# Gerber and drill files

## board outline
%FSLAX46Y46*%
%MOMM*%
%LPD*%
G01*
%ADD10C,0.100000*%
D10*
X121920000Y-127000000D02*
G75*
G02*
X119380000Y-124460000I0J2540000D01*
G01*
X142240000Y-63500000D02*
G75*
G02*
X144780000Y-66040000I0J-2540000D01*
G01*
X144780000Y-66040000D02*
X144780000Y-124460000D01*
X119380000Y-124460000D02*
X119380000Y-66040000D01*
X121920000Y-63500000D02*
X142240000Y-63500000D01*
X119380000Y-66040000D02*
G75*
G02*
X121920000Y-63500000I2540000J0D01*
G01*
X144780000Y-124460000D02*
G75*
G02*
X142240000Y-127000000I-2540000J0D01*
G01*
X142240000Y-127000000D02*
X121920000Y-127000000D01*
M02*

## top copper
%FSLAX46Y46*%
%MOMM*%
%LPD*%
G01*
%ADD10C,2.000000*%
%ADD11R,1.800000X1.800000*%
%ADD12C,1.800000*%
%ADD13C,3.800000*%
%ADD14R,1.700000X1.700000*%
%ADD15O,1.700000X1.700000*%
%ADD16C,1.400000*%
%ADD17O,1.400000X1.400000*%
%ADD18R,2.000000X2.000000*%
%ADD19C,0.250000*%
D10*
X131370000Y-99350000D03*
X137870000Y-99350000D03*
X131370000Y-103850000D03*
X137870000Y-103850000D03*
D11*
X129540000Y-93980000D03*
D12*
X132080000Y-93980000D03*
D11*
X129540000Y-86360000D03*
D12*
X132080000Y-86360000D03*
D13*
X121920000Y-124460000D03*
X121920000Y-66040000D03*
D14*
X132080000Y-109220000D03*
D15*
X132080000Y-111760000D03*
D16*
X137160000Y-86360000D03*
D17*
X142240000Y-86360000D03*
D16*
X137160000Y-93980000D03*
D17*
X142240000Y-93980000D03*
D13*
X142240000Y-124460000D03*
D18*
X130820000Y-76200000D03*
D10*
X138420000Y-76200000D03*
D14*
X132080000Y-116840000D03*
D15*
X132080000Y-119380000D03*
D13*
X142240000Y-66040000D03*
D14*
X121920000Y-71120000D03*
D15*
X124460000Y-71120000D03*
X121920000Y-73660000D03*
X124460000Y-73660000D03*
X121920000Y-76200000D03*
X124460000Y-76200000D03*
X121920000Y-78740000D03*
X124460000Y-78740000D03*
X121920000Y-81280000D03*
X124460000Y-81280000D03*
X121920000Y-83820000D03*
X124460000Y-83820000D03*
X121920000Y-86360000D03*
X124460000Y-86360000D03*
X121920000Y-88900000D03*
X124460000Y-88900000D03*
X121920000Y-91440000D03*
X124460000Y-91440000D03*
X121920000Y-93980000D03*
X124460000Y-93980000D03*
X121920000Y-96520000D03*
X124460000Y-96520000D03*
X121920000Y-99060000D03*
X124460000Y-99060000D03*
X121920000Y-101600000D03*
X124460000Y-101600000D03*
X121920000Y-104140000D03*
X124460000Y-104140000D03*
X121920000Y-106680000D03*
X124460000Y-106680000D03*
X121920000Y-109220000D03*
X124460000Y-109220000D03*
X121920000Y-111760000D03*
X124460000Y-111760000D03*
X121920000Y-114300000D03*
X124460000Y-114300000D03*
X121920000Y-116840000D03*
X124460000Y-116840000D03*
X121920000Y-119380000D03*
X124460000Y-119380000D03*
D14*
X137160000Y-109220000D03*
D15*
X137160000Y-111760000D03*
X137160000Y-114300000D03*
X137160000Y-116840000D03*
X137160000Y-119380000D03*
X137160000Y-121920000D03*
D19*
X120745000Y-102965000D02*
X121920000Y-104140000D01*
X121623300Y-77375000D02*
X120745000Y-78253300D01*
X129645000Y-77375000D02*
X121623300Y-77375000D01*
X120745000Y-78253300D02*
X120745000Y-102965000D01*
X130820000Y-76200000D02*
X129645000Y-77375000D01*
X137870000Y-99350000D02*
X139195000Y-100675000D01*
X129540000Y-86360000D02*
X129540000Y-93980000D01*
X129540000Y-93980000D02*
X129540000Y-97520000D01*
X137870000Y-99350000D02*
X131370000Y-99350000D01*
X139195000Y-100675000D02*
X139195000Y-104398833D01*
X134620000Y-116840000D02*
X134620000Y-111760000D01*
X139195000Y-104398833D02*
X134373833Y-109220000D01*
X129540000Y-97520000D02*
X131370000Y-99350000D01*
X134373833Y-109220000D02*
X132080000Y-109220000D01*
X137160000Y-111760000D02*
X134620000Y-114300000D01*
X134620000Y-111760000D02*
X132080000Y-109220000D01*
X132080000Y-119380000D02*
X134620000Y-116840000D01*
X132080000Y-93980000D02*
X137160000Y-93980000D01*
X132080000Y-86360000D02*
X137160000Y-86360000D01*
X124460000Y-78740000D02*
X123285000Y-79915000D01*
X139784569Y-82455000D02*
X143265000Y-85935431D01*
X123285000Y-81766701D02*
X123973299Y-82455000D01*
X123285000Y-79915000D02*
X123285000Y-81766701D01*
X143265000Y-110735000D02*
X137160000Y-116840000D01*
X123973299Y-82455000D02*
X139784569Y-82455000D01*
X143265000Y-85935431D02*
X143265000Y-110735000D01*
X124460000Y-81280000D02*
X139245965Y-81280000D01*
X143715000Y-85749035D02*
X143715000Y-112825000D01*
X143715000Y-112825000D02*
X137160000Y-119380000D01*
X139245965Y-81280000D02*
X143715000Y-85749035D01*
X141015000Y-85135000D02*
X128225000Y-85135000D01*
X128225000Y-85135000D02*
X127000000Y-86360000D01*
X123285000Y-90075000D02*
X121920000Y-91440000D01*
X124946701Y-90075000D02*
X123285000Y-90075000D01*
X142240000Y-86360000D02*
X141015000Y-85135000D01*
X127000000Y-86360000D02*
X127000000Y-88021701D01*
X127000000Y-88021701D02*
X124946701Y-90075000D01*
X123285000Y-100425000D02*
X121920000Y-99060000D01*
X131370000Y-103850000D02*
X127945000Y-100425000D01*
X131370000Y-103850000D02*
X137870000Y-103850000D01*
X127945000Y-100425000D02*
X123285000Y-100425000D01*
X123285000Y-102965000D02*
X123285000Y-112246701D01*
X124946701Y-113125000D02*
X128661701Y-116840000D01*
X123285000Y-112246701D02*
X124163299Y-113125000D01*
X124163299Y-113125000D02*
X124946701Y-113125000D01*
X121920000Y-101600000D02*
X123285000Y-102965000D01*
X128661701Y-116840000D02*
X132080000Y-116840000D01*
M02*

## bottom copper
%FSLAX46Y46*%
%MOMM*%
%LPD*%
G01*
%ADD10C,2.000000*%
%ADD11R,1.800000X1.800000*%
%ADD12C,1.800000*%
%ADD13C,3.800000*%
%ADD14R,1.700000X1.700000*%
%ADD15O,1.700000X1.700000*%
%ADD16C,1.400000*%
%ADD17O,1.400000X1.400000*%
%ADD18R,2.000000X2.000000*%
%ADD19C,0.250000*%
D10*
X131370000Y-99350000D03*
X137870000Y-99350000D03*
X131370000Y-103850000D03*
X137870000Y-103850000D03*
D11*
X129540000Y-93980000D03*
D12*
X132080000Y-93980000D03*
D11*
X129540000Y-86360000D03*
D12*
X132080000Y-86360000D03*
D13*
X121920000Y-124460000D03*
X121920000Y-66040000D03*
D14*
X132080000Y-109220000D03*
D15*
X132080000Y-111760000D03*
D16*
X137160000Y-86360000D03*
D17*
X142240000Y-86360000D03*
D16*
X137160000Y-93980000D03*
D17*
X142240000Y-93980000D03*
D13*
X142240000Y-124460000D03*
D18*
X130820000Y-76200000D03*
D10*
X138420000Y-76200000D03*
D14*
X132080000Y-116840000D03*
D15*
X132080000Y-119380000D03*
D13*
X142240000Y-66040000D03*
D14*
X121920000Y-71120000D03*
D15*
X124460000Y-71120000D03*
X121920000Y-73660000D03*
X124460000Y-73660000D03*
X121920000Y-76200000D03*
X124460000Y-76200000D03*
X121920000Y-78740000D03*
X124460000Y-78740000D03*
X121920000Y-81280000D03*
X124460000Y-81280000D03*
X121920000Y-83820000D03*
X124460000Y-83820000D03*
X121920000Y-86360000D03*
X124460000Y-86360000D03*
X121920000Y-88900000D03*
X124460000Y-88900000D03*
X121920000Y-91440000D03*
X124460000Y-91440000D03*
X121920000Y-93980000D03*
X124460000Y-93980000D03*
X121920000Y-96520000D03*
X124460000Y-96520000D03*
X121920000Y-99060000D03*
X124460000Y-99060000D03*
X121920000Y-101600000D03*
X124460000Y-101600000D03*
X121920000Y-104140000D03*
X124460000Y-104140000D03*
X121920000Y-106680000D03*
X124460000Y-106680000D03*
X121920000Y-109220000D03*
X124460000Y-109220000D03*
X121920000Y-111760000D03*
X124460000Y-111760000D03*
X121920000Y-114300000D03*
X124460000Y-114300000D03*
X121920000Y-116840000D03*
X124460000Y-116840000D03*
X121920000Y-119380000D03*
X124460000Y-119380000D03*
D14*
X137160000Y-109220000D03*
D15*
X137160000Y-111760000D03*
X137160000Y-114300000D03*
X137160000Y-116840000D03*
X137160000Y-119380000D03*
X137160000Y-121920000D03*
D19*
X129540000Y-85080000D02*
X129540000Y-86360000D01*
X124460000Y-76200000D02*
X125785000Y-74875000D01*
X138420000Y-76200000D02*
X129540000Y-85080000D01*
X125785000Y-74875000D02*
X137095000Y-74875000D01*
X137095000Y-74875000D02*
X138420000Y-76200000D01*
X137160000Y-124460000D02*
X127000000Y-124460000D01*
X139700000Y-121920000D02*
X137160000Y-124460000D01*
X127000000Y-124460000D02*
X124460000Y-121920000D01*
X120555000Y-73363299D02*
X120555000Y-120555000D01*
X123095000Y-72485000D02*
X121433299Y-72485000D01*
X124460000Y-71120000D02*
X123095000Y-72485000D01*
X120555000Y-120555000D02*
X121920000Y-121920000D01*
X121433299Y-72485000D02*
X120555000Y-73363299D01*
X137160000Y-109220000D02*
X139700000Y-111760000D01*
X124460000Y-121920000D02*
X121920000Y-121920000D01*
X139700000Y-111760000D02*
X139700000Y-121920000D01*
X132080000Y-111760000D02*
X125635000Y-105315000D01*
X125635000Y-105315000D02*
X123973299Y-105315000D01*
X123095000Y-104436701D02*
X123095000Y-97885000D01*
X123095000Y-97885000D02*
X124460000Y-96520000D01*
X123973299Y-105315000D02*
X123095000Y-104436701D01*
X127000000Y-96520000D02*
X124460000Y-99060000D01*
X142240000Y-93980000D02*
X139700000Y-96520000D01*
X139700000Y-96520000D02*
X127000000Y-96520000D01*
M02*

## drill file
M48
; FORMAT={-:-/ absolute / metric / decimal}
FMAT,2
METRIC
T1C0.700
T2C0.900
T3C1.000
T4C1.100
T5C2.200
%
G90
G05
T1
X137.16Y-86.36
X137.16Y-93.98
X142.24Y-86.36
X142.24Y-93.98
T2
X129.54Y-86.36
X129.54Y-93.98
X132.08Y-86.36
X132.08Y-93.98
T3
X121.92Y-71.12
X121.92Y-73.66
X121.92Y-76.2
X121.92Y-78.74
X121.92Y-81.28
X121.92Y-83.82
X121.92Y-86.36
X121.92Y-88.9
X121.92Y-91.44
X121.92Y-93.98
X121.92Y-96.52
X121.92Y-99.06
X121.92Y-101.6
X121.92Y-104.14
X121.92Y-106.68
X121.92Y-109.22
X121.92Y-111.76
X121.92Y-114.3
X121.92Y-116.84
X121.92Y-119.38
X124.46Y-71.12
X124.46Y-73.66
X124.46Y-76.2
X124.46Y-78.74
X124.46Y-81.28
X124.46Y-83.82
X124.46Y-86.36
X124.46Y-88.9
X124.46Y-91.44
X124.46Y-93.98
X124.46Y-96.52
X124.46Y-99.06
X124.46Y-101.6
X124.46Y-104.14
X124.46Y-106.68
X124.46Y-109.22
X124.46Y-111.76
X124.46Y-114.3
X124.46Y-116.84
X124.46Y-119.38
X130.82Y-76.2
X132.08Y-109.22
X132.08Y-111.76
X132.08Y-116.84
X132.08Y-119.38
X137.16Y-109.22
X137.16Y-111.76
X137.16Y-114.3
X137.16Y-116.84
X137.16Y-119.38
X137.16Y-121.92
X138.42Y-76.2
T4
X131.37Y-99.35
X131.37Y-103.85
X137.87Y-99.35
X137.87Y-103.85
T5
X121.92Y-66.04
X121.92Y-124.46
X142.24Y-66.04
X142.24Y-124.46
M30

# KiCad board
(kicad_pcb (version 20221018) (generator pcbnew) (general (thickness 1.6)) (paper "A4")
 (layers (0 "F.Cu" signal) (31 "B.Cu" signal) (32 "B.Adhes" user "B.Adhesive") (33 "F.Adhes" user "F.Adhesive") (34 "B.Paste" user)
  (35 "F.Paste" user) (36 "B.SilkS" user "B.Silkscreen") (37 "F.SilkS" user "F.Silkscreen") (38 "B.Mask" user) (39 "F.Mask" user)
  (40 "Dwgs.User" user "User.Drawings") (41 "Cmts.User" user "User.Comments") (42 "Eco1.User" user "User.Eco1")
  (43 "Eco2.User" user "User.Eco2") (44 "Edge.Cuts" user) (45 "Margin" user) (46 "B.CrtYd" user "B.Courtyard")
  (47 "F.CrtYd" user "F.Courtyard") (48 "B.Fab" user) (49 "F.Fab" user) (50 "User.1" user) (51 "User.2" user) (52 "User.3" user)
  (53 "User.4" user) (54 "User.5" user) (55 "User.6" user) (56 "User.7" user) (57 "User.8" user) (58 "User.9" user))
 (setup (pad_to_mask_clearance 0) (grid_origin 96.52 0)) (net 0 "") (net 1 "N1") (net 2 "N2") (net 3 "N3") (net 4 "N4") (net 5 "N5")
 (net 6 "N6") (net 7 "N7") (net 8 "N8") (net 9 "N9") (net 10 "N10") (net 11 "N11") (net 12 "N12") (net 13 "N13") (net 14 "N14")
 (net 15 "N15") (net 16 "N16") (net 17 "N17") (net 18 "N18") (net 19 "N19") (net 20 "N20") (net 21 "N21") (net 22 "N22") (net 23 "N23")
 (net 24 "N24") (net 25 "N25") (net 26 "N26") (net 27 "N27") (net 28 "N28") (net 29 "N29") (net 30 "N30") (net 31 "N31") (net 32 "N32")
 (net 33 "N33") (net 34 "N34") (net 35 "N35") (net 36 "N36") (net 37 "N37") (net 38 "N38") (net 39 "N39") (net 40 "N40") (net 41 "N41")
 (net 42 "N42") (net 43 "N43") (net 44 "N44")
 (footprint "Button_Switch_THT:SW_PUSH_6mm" (layer "F.Cu") (at 131.37 99.35)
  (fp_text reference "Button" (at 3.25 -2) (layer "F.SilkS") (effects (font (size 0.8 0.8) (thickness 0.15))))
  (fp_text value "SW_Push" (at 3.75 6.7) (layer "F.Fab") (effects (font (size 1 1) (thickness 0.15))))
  (pad "1" thru_hole circle (at 0 0 90) (size 2 2) (drill 1.1) (layers "*.Cu" "*.Mask") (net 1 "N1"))
  (pad "1" thru_hole circle (at 6.5 0 90) (size 2 2) (drill 1.1) (layers "*.Cu" "*.Mask") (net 1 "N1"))
  (pad "2" thru_hole circle (at 0 4.5 90) (size 2 2) (drill 1.1) (layers "*.Cu" "*.Mask") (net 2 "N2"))
  (pad "2" thru_hole circle (at 6.5 4.5 90) (size 2 2) (drill 1.1) (layers "*.Cu" "*.Mask") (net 2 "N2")))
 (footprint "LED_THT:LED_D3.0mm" (layer "F.Cu") (at 129.54 93.98)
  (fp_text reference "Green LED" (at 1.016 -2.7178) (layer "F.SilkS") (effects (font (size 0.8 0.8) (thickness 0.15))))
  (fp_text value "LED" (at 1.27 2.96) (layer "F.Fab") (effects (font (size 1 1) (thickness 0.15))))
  (pad "1" thru_hole rect (at 0 0) (size 1.8 1.8) (drill 0.9) (layers "*.Cu" "*.Mask") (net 1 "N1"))
  (pad "2" thru_hole circle (at 2.54 0) (size 1.8 1.8) (drill 0.9) (layers "*.Cu" "*.Mask") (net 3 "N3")))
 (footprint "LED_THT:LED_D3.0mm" (layer "F.Cu") (at 129.54 86.36)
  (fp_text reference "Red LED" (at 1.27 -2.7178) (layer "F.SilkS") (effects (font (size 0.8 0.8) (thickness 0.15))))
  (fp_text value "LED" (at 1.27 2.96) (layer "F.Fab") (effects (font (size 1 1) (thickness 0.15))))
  (pad "1" thru_hole rect (at 0 0) (size 1.8 1.8) (drill 0.9) (layers "*.Cu" "*.Mask") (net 1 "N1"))
  (pad "2" thru_hole circle (at 2.54 0) (size 1.8 1.8) (drill 0.9) (layers "*.Cu" "*.Mask") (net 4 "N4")))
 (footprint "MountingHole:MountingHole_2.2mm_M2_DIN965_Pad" (layer "F.Cu") (at 121.92 124.46)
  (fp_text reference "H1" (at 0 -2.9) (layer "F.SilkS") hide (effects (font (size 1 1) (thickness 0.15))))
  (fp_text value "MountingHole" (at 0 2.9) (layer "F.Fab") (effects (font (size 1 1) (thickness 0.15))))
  (pad "1" thru_hole circle (at 0 0) (size 3.8 3.8) (drill 2.2) (layers "*.Cu" "*.Mask")))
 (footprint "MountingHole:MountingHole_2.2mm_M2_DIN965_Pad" (layer "F.Cu") (at 121.92 66.04)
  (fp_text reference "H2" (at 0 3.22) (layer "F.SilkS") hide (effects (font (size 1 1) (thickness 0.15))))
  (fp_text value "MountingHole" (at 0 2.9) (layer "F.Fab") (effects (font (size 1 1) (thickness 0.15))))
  (pad "1" thru_hole circle (at 0 0) (size 3.8 3.8) (drill 2.2) (layers "*.Cu" "*.Mask")))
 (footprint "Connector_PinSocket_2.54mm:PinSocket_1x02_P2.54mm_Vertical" (layer "F.Cu") (at 132.08 109.22)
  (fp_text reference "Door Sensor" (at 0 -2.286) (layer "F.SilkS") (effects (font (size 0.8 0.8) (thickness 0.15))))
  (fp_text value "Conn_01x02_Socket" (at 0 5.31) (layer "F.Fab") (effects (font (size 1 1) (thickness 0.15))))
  (pad "1" thru_hole rect (at 0 0) (size 1.7 1.7) (drill 1) (layers "*.Cu" "*.Mask") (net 1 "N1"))
  (pad "2" thru_hole oval (at 0 2.54) (size 1.7 1.7) (drill 1) (layers "*.Cu" "*.Mask") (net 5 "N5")))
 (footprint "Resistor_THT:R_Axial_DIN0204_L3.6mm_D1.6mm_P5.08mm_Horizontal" (layer "F.Cu") (at 137.16 86.36)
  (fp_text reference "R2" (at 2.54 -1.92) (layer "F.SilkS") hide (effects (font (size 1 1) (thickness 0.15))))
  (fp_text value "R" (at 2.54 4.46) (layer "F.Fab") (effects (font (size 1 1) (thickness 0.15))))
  (pad "1" thru_hole circle (at 0 0) (size 1.4 1.4) (drill 0.7) (layers "*.Cu" "*.Mask") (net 4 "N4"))
  (pad "2" thru_hole oval (at 5.08 0) (size 1.4 1.4) (drill 0.7) (layers "*.Cu" "*.Mask") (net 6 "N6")))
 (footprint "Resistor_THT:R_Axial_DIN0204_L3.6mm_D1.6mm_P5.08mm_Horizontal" (layer "F.Cu") (at 137.16 93.98)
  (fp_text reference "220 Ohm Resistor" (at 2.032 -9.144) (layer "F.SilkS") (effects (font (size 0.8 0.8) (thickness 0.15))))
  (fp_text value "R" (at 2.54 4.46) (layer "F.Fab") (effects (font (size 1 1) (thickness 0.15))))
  (pad "1" thru_hole circle (at 0 0) (size 1.4 1.4) (drill 0.7) (layers "*.Cu" "*.Mask") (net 3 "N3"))
  (pad "2" thru_hole oval (at 5.08 0) (size 1.4 1.4) (drill 0.7) (layers "*.Cu" "*.Mask") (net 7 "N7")))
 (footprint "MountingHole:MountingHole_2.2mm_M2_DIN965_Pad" (layer "F.Cu") (at 142.24 124.46)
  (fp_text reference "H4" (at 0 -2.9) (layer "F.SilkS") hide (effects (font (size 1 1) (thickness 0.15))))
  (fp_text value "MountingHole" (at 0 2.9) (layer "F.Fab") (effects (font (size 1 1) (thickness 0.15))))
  (pad "1" thru_hole circle (at 0 0) (size 3.8 3.8) (drill 2.2) (layers "*.Cu" "*.Mask")))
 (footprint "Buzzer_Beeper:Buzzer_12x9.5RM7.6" (layer "F.Cu") (at 130.82 76.2)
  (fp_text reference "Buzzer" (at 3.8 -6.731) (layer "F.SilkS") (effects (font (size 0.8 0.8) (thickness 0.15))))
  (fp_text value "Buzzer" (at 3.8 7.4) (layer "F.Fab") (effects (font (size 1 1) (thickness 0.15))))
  (pad "1" thru_hole rect (at 0 0) (size 2 2) (drill 1) (layers "*.Cu" "*.Mask") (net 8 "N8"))
  (pad "2" thru_hole circle (at 7.6 0) (size 2 2) (drill 1) (layers "*.Cu" "*.Mask") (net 1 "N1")))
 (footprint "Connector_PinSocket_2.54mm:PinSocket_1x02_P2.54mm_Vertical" (layer "F.Cu") (at 132.08 116.84)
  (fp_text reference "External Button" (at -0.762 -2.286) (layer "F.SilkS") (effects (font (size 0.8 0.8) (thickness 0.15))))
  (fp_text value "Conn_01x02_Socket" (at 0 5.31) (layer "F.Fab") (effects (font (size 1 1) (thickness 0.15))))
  (pad "1" thru_hole rect (at 0 0) (size 1.7 1.7) (drill 1) (layers "*.Cu" "*.Mask") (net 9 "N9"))
  (pad "2" thru_hole oval (at 0 2.54) (size 1.7 1.7) (drill 1) (layers "*.Cu" "*.Mask") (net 1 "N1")))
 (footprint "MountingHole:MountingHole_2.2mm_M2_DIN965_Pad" (layer "F.Cu") (at 142.24 66.04)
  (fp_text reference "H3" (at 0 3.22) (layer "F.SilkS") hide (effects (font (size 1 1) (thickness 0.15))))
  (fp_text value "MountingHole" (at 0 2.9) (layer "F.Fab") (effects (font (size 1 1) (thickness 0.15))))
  (pad "1" thru_hole circle (at 0 0) (size 3.8 3.8) (drill 2.2) (layers "*.Cu" "*.Mask")))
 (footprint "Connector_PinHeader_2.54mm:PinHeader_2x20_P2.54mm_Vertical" (layer "F.Cu") (at 121.92 71.12)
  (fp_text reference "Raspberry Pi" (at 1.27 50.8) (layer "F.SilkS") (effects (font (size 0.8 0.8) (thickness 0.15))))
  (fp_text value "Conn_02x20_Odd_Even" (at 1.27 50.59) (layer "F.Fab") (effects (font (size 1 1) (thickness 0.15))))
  (pad "1" thru_hole rect (at 0 0) (size 1.7 1.7) (drill 1) (layers "*.Cu" "*.Mask") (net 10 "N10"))
  (pad "2" thru_hole oval (at 2.54 0) (size 1.7 1.7) (drill 1) (layers "*.Cu" "*.Mask") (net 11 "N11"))
  (pad "3" thru_hole oval (at 0 2.54) (size 1.7 1.7) (drill 1) (layers "*.Cu" "*.Mask") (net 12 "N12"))
  (pad "4" thru_hole oval (at 2.54 2.54) (size 1.7 1.7) (drill 1) (layers "*.Cu" "*.Mask") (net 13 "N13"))
  (pad "5" thru_hole oval (at 0 5.08) (size 1.7 1.7) (drill 1) (layers "*.Cu" "*.Mask") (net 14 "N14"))
  (pad "6" thru_hole oval (at 2.54 5.08) (size 1.7 1.7) (drill 1) (layers "*.Cu" "*.Mask") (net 1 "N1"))
  (pad "7" thru_hole oval (at 0 7.62) (size 1.7 1.7) (drill 1) (layers "*.Cu" "*.Mask") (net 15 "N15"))
  (pad "8" thru_hole oval (at 2.54 7.62) (size 1.7 1.7) (drill 1) (layers "*.Cu" "*.Mask") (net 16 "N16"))
  (pad "9" thru_hole oval (at 0 10.16) (size 1.7 1.7) (drill 1) (layers "*.Cu" "*.Mask") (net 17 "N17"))
  (pad "10" thru_hole oval (at 2.54 10.16) (size 1.7 1.7) (drill 1) (layers "*.Cu" "*.Mask") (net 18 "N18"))
  (pad "11" thru_hole oval (at 0 12.7) (size 1.7 1.7) (drill 1) (layers "*.Cu" "*.Mask") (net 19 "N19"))
  (pad "12" thru_hole oval (at 2.54 12.7) (size 1.7 1.7) (drill 1) (layers "*.Cu" "*.Mask") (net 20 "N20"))
  (pad "13" thru_hole oval (at 0 15.24) (size 1.7 1.7) (drill 1) (layers "*.Cu" "*.Mask") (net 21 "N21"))
  (pad "14" thru_hole oval (at 2.54 15.24) (size 1.7 1.7) (drill 1) (layers "*.Cu" "*.Mask") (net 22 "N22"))
  (pad "15" thru_hole oval (at 0 17.78) (size 1.7 1.7) (drill 1) (layers "*.Cu" "*.Mask") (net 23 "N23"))
  (pad "16" thru_hole oval (at 2.54 17.78) (size 1.7 1.7) (drill 1) (layers "*.Cu" "*.Mask") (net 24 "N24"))
  (pad "17" thru_hole oval (at 0 20.32) (size 1.7 1.7) (drill 1) (layers "*.Cu" "*.Mask") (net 6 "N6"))
  (pad "18" thru_hole oval (at 2.54 20.32) (size 1.7 1.7) (drill 1) (layers "*.Cu" "*.Mask") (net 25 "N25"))
  (pad "19" thru_hole oval (at 0 22.86) (size 1.7 1.7) (drill 1) (layers "*.Cu" "*.Mask") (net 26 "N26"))
  (pad "20" thru_hole oval (at 2.54 22.86) (size 1.7 1.7) (drill 1) (layers "*.Cu" "*.Mask") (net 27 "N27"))
  (pad "21" thru_hole oval (at 0 25.4) (size 1.7 1.7) (drill 1) (layers "*.Cu" "*.Mask") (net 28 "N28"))
  (pad "22" thru_hole oval (at 2.54 25.4) (size 1.7 1.7) (drill 1) (layers "*.Cu" "*.Mask") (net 5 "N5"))
  (pad "23" thru_hole oval (at 0 27.94) (size 1.7 1.7) (drill 1) (layers "*.Cu" "*.Mask") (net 2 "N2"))
  (pad "24" thru_hole oval (at 2.54 27.94) (size 1.7 1.7) (drill 1) (layers "*.Cu" "*.Mask") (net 7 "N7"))
  (pad "25" thru_hole oval (at 0 30.48) (size 1.7 1.7) (drill 1) (layers "*.Cu" "*.Mask") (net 9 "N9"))
  (pad "26" thru_hole oval (at 2.54 30.48) (size 1.7 1.7) (drill 1) (layers "*.Cu" "*.Mask") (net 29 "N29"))
  (pad "27" thru_hole oval (at 0 33.02) (size 1.7 1.7) (drill 1) (layers "*.Cu" "*.Mask") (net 8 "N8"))
  (pad "28" thru_hole oval (at 2.54 33.02) (size 1.7 1.7) (drill 1) (layers "*.Cu" "*.Mask") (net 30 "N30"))
  (pad "29" thru_hole oval (at 0 35.56) (size 1.7 1.7) (drill 1) (layers "*.Cu" "*.Mask") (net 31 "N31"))
  (pad "30" thru_hole oval (at 2.54 35.56) (size 1.7 1.7) (drill 1) (layers "*.Cu" "*.Mask") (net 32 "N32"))
  (pad "31" thru_hole oval (at 0 38.1) (size 1.7 1.7) (drill 1) (layers "*.Cu" "*.Mask") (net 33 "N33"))
  (pad "32" thru_hole oval (at 2.54 38.1) (size 1.7 1.7) (drill 1) (layers "*.Cu" "*.Mask") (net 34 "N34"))
  (pad "33" thru_hole oval (at 0 40.64) (size 1.7 1.7) (drill 1) (layers "*.Cu" "*.Mask") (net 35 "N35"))
  (pad "34" thru_hole oval (at 2.54 40.64) (size 1.7 1.7) (drill 1) (layers "*.Cu" "*.Mask") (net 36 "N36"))
  (pad "35" thru_hole oval (at 0 43.18) (size 1.7 1.7) (drill 1) (layers "*.Cu" "*.Mask") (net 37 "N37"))
  (pad "36" thru_hole oval (at 2.54 43.18) (size 1.7 1.7) (drill 1) (layers "*.Cu" "*.Mask") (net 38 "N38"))
  (pad "37" thru_hole oval (at 0 45.72) (size 1.7 1.7) (drill 1) (layers "*.Cu" "*.Mask") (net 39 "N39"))
  (pad "38" thru_hole oval (at 2.54 45.72) (size 1.7 1.7) (drill 1) (layers "*.Cu" "*.Mask") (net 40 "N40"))
  (pad "39" thru_hole oval (at 0 48.26) (size 1.7 1.7) (drill 1) (layers "*.Cu" "*.Mask") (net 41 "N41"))
  (pad "40" thru_hole oval (at 2.54 48.26) (size 1.7 1.7) (drill 1) (layers "*.Cu" "*.Mask") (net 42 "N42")))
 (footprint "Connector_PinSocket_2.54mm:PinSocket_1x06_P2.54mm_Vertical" (layer "B.Cu") (at 137.16 109.22 180)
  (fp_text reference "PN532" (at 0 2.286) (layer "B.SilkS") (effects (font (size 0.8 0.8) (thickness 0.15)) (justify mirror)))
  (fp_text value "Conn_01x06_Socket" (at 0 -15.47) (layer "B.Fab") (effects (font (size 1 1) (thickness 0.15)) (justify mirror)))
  (pad "1" thru_hole rect (at 0 0 180) (size 1.7 1.7) (drill 1) (layers "*.Cu" "*.Mask") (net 11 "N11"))
  (pad "2" thru_hole oval (at 0 -2.54 180) (size 1.7 1.7) (drill 1) (layers "*.Cu" "*.Mask") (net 1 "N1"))
  (pad "3" thru_hole oval (at 0 -5.08 180) (size 1.7 1.7) (drill 1) (layers "*.Cu" "*.Mask") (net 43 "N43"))
  (pad "4" thru_hole oval (at 0 -7.62 180) (size 1.7 1.7) (drill 1) (layers "*.Cu" "*.Mask") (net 16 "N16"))
  (pad "5" thru_hole oval (at 0 -10.16 180) (size 1.7 1.7) (drill 1) (layers "*.Cu" "*.Mask") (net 18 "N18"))
  (pad "6" thru_hole oval (at 0 -12.7 180) (size 1.7 1.7) (drill 1) (layers "*.Cu" "*.Mask") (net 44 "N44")))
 (gr_arc (start 121.92 127) (mid 120.123949 126.256051) (end 119.38 124.46) (stroke (width 0.1) (type default)) (layer "Edge.Cuts"))
 (gr_arc (start 142.24 63.5) (mid 144.036051 64.243949) (end 144.78 66.04) (stroke (width 0.1) (type default)) (layer "Edge.Cuts"))
 (gr_line (start 144.78 66.04) (end 144.78 124.46) (stroke (width 0.1) (type default)) (layer "Edge.Cuts"))
 (gr_line (start 119.38 124.46) (end 119.38 66.04) (stroke (width 0.1) (type default)) (layer "Edge.Cuts"))
 (gr_line (start 121.92 63.5) (end 142.24 63.5) (stroke (width 0.1) (type default)) (layer "Edge.Cuts"))
 (gr_arc (start 119.38 66.04) (mid 120.123949 64.243949) (end 121.92 63.5) (stroke (width 0.1) (type default)) (layer "Edge.Cuts"))
 (gr_arc (start 144.78 124.46) (mid 144.036051 126.256051) (end 142.24 127) (stroke (width 0.1) (type default)) (layer "Edge.Cuts"))
 (gr_line (start 142.24 127) (end 121.92 127) (stroke (width 0.1) (type default)) (layer "Edge.Cuts"))
 (segment (start 120.745 102.965) (end 121.92 104.14) (width 0.25) (layer "F.Cu") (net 8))
 (segment (start 121.6233 77.375) (end 120.745 78.2533) (width 0.25) (layer "F.Cu") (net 8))
 (segment (start 129.645 77.375) (end 121.6233 77.375) (width 0.25) (layer "F.Cu") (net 8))
 (segment (start 120.745 78.2533) (end 120.745 102.965) (width 0.25) (layer "F.Cu") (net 8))
 (segment (start 130.82 76.2) (end 129.645 77.375) (width 0.25) (layer "F.Cu") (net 8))
 (segment (start 137.87 99.35) (end 139.195 100.675) (width 0.25) (layer "F.Cu") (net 1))
 (segment (start 129.54 86.36) (end 129.54 93.98) (width 0.25) (layer "F.Cu") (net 1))
 (segment (start 129.54 93.98) (end 129.54 97.52) (width 0.25) (layer "F.Cu") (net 1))
 (segment (start 137.87 99.35) (end 131.37 99.35) (width 0.25) (layer "F.Cu") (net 1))
 (segment (start 139.195 100.675) (end 139.195 104.398833) (width 0.25) (layer "F.Cu") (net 1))
 (segment (start 134.62 116.84) (end 134.62 111.76) (width 0.25) (layer "F.Cu") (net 1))
 (segment (start 139.195 104.398833) (end 134.373833 109.22) (width 0.25) (layer "F.Cu") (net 1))
 (segment (start 129.54 97.52) (end 131.37 99.35) (width 0.25) (layer "F.Cu") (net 1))
 (segment (start 134.373833 109.22) (end 132.08 109.22) (width 0.25) (layer "F.Cu") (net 1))
 (segment (start 137.16 111.76) (end 134.62 114.3) (width 0.25) (layer "F.Cu") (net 1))
 (segment (start 134.62 111.76) (end 132.08 109.22) (width 0.25) (layer "F.Cu") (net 1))
 (segment (start 132.08 119.38) (end 134.62 116.84) (width 0.25) (layer "F.Cu") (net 1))
 (segment (start 129.54 85.08) (end 129.54 86.36) (width 0.25) (layer "B.Cu") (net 1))
 (segment (start 124.46 76.2) (end 125.785 74.875) (width 0.25) (layer "B.Cu") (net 1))
 (segment (start 138.42 76.2) (end 129.54 85.08) (width 0.25) (layer "B.Cu") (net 1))
 (segment (start 125.785 74.875) (end 137.095 74.875) (width 0.25) (layer "B.Cu") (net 1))
 (segment (start 137.095 74.875) (end 138.42 76.2) (width 0.25) (layer "B.Cu") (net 1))
 (segment (start 132.08 93.98) (end 137.16 93.98) (width 0.25) (layer "F.Cu") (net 3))
 (segment (start 132.08 86.36) (end 137.16 86.36) (width 0.25) (layer "F.Cu") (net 4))
 (segment (start 137.16 124.46) (end 127 124.46) (width 0.25) (layer "B.Cu") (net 11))
 (segment (start 139.7 121.92) (end 137.16 124.46) (width 0.25) (layer "B.Cu") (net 11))
 (segment (start 127 124.46) (end 124.46 121.92) (width 0.25) (layer "B.Cu") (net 11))
 (segment (start 120.555 73.363299) (end 120.555 120.555) (width 0.25) (layer "B.Cu") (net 11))
 (segment (start 123.095 72.485) (end 121.433299 72.485) (width 0.25) (layer "B.Cu") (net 11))
 (segment (start 124.46 71.12) (end 123.095 72.485) (width 0.25) (layer "B.Cu") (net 11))
 (segment (start 120.555 120.555) (end 121.92 121.92) (width 0.25) (layer "B.Cu") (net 11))
 (segment (start 121.433299 72.485) (end 120.555 73.363299) (width 0.25) (layer "B.Cu") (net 11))
 (segment (start 137.16 109.22) (end 139.7 111.76) (width 0.25) (layer "B.Cu") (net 11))
 (segment (start 124.46 121.92) (end 121.92 121.92) (width 0.25) (layer "B.Cu") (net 11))
 (segment (start 139.7 111.76) (end 139.7 121.92) (width 0.25) (layer "B.Cu") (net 11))
 (segment (start 124.46 78.74) (end 123.285 79.915) (width 0.25) (layer "F.Cu") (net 16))
 (segment (start 139.784569 82.455) (end 143.265 85.935431) (width 0.25) (layer "F.Cu") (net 16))
 (segment (start 123.285 81.766701) (end 123.973299 82.455) (width 0.25) (layer "F.Cu") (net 16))
 (segment (start 123.285 79.915) (end 123.285 81.766701) (width 0.25) (layer "F.Cu") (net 16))
 (segment (start 143.265 110.735) (end 137.16 116.84) (width 0.25) (layer "F.Cu") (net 16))
 (segment (start 123.973299 82.455) (end 139.784569 82.455) (width 0.25) (layer "F.Cu") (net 16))
 (segment (start 143.265 85.935431) (end 143.265 110.735) (width 0.25) (layer "F.Cu") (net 16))
 (segment (start 124.46 81.28) (end 139.245965 81.28) (width 0.25) (layer "F.Cu") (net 18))
 (segment (start 143.715 85.749035) (end 143.715 112.825) (width 0.25) (layer "F.Cu") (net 18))
 (segment (start 143.715 112.825) (end 137.16 119.38) (width 0.25) (layer "F.Cu") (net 18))
 (segment (start 139.245965 81.28) (end 143.715 85.749035) (width 0.25) (layer "F.Cu") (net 18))
 (segment (start 141.015 85.135) (end 128.225 85.135) (width 0.25) (layer "F.Cu") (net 6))
 (segment (start 128.225 85.135) (end 127 86.36) (width 0.25) (layer "F.Cu") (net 6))
 (segment (start 123.285 90.075) (end 121.92 91.44) (width 0.25) (layer "F.Cu") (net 6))
 (segment (start 124.946701 90.075) (end 123.285 90.075) (width 0.25) (layer "F.Cu") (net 6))
 (segment (start 142.24 86.36) (end 141.015 85.135) (width 0.25) (layer "F.Cu") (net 6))
 (segment (start 127 86.36) (end 127 88.021701) (width 0.25) (layer "F.Cu") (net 6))
 (segment (start 127 88.021701) (end 124.946701 90.075) (width 0.25) (layer "F.Cu") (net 6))
 (segment (start 132.08 111.76) (end 125.635 105.315) (width 0.25) (layer "B.Cu") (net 5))
 (segment (start 125.635 105.315) (end 123.973299 105.315) (width 0.25) (layer "B.Cu") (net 5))
 (segment (start 123.095 104.436701) (end 123.095 97.885) (width 0.25) (layer "B.Cu") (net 5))
 (segment (start 123.095 97.885) (end 124.46 96.52) (width 0.25) (layer "B.Cu") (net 5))
 (segment (start 123.973299 105.315) (end 123.095 104.436701) (width 0.25) (layer "B.Cu") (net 5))
 (segment (start 123.285 100.425) (end 121.92 99.06) (width 0.25) (layer "F.Cu") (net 2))
 (segment (start 131.37 103.85) (end 127.945 100.425) (width 0.25) (layer "F.Cu") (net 2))
 (segment (start 131.37 103.85) (end 137.87 103.85) (width 0.25) (layer "F.Cu") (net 2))
 (segment (start 127.945 100.425) (end 123.285 100.425) (width 0.25) (layer "F.Cu") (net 2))
 (segment (start 123.285 102.965) (end 123.285 112.246701) (width 0.25) (layer "F.Cu") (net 9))
 (segment (start 124.946701 113.125) (end 128.661701 116.84) (width 0.25) (layer "F.Cu") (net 9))
 (segment (start 123.285 112.246701) (end 124.163299 113.125) (width 0.25) (layer "F.Cu") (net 9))
 (segment (start 124.163299 113.125) (end 124.946701 113.125) (width 0.25) (layer "F.Cu") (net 9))
 (segment (start 121.92 101.6) (end 123.285 102.965) (width 0.25) (layer "F.Cu") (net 9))
 (segment (start 128.661701 116.84) (end 132.08 116.84) (width 0.25) (layer "F.Cu") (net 9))
 (segment (start 127 96.52) (end 124.46 99.06) (width 0.25) (layer "B.Cu") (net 7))
 (segment (start 142.24 93.98) (end 139.7 96.52) (width 0.25) (layer "B.Cu") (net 7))
 (segment (start 139.7 96.52) (end 127 96.52) (width 0.25) (layer "B.Cu") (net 7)))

